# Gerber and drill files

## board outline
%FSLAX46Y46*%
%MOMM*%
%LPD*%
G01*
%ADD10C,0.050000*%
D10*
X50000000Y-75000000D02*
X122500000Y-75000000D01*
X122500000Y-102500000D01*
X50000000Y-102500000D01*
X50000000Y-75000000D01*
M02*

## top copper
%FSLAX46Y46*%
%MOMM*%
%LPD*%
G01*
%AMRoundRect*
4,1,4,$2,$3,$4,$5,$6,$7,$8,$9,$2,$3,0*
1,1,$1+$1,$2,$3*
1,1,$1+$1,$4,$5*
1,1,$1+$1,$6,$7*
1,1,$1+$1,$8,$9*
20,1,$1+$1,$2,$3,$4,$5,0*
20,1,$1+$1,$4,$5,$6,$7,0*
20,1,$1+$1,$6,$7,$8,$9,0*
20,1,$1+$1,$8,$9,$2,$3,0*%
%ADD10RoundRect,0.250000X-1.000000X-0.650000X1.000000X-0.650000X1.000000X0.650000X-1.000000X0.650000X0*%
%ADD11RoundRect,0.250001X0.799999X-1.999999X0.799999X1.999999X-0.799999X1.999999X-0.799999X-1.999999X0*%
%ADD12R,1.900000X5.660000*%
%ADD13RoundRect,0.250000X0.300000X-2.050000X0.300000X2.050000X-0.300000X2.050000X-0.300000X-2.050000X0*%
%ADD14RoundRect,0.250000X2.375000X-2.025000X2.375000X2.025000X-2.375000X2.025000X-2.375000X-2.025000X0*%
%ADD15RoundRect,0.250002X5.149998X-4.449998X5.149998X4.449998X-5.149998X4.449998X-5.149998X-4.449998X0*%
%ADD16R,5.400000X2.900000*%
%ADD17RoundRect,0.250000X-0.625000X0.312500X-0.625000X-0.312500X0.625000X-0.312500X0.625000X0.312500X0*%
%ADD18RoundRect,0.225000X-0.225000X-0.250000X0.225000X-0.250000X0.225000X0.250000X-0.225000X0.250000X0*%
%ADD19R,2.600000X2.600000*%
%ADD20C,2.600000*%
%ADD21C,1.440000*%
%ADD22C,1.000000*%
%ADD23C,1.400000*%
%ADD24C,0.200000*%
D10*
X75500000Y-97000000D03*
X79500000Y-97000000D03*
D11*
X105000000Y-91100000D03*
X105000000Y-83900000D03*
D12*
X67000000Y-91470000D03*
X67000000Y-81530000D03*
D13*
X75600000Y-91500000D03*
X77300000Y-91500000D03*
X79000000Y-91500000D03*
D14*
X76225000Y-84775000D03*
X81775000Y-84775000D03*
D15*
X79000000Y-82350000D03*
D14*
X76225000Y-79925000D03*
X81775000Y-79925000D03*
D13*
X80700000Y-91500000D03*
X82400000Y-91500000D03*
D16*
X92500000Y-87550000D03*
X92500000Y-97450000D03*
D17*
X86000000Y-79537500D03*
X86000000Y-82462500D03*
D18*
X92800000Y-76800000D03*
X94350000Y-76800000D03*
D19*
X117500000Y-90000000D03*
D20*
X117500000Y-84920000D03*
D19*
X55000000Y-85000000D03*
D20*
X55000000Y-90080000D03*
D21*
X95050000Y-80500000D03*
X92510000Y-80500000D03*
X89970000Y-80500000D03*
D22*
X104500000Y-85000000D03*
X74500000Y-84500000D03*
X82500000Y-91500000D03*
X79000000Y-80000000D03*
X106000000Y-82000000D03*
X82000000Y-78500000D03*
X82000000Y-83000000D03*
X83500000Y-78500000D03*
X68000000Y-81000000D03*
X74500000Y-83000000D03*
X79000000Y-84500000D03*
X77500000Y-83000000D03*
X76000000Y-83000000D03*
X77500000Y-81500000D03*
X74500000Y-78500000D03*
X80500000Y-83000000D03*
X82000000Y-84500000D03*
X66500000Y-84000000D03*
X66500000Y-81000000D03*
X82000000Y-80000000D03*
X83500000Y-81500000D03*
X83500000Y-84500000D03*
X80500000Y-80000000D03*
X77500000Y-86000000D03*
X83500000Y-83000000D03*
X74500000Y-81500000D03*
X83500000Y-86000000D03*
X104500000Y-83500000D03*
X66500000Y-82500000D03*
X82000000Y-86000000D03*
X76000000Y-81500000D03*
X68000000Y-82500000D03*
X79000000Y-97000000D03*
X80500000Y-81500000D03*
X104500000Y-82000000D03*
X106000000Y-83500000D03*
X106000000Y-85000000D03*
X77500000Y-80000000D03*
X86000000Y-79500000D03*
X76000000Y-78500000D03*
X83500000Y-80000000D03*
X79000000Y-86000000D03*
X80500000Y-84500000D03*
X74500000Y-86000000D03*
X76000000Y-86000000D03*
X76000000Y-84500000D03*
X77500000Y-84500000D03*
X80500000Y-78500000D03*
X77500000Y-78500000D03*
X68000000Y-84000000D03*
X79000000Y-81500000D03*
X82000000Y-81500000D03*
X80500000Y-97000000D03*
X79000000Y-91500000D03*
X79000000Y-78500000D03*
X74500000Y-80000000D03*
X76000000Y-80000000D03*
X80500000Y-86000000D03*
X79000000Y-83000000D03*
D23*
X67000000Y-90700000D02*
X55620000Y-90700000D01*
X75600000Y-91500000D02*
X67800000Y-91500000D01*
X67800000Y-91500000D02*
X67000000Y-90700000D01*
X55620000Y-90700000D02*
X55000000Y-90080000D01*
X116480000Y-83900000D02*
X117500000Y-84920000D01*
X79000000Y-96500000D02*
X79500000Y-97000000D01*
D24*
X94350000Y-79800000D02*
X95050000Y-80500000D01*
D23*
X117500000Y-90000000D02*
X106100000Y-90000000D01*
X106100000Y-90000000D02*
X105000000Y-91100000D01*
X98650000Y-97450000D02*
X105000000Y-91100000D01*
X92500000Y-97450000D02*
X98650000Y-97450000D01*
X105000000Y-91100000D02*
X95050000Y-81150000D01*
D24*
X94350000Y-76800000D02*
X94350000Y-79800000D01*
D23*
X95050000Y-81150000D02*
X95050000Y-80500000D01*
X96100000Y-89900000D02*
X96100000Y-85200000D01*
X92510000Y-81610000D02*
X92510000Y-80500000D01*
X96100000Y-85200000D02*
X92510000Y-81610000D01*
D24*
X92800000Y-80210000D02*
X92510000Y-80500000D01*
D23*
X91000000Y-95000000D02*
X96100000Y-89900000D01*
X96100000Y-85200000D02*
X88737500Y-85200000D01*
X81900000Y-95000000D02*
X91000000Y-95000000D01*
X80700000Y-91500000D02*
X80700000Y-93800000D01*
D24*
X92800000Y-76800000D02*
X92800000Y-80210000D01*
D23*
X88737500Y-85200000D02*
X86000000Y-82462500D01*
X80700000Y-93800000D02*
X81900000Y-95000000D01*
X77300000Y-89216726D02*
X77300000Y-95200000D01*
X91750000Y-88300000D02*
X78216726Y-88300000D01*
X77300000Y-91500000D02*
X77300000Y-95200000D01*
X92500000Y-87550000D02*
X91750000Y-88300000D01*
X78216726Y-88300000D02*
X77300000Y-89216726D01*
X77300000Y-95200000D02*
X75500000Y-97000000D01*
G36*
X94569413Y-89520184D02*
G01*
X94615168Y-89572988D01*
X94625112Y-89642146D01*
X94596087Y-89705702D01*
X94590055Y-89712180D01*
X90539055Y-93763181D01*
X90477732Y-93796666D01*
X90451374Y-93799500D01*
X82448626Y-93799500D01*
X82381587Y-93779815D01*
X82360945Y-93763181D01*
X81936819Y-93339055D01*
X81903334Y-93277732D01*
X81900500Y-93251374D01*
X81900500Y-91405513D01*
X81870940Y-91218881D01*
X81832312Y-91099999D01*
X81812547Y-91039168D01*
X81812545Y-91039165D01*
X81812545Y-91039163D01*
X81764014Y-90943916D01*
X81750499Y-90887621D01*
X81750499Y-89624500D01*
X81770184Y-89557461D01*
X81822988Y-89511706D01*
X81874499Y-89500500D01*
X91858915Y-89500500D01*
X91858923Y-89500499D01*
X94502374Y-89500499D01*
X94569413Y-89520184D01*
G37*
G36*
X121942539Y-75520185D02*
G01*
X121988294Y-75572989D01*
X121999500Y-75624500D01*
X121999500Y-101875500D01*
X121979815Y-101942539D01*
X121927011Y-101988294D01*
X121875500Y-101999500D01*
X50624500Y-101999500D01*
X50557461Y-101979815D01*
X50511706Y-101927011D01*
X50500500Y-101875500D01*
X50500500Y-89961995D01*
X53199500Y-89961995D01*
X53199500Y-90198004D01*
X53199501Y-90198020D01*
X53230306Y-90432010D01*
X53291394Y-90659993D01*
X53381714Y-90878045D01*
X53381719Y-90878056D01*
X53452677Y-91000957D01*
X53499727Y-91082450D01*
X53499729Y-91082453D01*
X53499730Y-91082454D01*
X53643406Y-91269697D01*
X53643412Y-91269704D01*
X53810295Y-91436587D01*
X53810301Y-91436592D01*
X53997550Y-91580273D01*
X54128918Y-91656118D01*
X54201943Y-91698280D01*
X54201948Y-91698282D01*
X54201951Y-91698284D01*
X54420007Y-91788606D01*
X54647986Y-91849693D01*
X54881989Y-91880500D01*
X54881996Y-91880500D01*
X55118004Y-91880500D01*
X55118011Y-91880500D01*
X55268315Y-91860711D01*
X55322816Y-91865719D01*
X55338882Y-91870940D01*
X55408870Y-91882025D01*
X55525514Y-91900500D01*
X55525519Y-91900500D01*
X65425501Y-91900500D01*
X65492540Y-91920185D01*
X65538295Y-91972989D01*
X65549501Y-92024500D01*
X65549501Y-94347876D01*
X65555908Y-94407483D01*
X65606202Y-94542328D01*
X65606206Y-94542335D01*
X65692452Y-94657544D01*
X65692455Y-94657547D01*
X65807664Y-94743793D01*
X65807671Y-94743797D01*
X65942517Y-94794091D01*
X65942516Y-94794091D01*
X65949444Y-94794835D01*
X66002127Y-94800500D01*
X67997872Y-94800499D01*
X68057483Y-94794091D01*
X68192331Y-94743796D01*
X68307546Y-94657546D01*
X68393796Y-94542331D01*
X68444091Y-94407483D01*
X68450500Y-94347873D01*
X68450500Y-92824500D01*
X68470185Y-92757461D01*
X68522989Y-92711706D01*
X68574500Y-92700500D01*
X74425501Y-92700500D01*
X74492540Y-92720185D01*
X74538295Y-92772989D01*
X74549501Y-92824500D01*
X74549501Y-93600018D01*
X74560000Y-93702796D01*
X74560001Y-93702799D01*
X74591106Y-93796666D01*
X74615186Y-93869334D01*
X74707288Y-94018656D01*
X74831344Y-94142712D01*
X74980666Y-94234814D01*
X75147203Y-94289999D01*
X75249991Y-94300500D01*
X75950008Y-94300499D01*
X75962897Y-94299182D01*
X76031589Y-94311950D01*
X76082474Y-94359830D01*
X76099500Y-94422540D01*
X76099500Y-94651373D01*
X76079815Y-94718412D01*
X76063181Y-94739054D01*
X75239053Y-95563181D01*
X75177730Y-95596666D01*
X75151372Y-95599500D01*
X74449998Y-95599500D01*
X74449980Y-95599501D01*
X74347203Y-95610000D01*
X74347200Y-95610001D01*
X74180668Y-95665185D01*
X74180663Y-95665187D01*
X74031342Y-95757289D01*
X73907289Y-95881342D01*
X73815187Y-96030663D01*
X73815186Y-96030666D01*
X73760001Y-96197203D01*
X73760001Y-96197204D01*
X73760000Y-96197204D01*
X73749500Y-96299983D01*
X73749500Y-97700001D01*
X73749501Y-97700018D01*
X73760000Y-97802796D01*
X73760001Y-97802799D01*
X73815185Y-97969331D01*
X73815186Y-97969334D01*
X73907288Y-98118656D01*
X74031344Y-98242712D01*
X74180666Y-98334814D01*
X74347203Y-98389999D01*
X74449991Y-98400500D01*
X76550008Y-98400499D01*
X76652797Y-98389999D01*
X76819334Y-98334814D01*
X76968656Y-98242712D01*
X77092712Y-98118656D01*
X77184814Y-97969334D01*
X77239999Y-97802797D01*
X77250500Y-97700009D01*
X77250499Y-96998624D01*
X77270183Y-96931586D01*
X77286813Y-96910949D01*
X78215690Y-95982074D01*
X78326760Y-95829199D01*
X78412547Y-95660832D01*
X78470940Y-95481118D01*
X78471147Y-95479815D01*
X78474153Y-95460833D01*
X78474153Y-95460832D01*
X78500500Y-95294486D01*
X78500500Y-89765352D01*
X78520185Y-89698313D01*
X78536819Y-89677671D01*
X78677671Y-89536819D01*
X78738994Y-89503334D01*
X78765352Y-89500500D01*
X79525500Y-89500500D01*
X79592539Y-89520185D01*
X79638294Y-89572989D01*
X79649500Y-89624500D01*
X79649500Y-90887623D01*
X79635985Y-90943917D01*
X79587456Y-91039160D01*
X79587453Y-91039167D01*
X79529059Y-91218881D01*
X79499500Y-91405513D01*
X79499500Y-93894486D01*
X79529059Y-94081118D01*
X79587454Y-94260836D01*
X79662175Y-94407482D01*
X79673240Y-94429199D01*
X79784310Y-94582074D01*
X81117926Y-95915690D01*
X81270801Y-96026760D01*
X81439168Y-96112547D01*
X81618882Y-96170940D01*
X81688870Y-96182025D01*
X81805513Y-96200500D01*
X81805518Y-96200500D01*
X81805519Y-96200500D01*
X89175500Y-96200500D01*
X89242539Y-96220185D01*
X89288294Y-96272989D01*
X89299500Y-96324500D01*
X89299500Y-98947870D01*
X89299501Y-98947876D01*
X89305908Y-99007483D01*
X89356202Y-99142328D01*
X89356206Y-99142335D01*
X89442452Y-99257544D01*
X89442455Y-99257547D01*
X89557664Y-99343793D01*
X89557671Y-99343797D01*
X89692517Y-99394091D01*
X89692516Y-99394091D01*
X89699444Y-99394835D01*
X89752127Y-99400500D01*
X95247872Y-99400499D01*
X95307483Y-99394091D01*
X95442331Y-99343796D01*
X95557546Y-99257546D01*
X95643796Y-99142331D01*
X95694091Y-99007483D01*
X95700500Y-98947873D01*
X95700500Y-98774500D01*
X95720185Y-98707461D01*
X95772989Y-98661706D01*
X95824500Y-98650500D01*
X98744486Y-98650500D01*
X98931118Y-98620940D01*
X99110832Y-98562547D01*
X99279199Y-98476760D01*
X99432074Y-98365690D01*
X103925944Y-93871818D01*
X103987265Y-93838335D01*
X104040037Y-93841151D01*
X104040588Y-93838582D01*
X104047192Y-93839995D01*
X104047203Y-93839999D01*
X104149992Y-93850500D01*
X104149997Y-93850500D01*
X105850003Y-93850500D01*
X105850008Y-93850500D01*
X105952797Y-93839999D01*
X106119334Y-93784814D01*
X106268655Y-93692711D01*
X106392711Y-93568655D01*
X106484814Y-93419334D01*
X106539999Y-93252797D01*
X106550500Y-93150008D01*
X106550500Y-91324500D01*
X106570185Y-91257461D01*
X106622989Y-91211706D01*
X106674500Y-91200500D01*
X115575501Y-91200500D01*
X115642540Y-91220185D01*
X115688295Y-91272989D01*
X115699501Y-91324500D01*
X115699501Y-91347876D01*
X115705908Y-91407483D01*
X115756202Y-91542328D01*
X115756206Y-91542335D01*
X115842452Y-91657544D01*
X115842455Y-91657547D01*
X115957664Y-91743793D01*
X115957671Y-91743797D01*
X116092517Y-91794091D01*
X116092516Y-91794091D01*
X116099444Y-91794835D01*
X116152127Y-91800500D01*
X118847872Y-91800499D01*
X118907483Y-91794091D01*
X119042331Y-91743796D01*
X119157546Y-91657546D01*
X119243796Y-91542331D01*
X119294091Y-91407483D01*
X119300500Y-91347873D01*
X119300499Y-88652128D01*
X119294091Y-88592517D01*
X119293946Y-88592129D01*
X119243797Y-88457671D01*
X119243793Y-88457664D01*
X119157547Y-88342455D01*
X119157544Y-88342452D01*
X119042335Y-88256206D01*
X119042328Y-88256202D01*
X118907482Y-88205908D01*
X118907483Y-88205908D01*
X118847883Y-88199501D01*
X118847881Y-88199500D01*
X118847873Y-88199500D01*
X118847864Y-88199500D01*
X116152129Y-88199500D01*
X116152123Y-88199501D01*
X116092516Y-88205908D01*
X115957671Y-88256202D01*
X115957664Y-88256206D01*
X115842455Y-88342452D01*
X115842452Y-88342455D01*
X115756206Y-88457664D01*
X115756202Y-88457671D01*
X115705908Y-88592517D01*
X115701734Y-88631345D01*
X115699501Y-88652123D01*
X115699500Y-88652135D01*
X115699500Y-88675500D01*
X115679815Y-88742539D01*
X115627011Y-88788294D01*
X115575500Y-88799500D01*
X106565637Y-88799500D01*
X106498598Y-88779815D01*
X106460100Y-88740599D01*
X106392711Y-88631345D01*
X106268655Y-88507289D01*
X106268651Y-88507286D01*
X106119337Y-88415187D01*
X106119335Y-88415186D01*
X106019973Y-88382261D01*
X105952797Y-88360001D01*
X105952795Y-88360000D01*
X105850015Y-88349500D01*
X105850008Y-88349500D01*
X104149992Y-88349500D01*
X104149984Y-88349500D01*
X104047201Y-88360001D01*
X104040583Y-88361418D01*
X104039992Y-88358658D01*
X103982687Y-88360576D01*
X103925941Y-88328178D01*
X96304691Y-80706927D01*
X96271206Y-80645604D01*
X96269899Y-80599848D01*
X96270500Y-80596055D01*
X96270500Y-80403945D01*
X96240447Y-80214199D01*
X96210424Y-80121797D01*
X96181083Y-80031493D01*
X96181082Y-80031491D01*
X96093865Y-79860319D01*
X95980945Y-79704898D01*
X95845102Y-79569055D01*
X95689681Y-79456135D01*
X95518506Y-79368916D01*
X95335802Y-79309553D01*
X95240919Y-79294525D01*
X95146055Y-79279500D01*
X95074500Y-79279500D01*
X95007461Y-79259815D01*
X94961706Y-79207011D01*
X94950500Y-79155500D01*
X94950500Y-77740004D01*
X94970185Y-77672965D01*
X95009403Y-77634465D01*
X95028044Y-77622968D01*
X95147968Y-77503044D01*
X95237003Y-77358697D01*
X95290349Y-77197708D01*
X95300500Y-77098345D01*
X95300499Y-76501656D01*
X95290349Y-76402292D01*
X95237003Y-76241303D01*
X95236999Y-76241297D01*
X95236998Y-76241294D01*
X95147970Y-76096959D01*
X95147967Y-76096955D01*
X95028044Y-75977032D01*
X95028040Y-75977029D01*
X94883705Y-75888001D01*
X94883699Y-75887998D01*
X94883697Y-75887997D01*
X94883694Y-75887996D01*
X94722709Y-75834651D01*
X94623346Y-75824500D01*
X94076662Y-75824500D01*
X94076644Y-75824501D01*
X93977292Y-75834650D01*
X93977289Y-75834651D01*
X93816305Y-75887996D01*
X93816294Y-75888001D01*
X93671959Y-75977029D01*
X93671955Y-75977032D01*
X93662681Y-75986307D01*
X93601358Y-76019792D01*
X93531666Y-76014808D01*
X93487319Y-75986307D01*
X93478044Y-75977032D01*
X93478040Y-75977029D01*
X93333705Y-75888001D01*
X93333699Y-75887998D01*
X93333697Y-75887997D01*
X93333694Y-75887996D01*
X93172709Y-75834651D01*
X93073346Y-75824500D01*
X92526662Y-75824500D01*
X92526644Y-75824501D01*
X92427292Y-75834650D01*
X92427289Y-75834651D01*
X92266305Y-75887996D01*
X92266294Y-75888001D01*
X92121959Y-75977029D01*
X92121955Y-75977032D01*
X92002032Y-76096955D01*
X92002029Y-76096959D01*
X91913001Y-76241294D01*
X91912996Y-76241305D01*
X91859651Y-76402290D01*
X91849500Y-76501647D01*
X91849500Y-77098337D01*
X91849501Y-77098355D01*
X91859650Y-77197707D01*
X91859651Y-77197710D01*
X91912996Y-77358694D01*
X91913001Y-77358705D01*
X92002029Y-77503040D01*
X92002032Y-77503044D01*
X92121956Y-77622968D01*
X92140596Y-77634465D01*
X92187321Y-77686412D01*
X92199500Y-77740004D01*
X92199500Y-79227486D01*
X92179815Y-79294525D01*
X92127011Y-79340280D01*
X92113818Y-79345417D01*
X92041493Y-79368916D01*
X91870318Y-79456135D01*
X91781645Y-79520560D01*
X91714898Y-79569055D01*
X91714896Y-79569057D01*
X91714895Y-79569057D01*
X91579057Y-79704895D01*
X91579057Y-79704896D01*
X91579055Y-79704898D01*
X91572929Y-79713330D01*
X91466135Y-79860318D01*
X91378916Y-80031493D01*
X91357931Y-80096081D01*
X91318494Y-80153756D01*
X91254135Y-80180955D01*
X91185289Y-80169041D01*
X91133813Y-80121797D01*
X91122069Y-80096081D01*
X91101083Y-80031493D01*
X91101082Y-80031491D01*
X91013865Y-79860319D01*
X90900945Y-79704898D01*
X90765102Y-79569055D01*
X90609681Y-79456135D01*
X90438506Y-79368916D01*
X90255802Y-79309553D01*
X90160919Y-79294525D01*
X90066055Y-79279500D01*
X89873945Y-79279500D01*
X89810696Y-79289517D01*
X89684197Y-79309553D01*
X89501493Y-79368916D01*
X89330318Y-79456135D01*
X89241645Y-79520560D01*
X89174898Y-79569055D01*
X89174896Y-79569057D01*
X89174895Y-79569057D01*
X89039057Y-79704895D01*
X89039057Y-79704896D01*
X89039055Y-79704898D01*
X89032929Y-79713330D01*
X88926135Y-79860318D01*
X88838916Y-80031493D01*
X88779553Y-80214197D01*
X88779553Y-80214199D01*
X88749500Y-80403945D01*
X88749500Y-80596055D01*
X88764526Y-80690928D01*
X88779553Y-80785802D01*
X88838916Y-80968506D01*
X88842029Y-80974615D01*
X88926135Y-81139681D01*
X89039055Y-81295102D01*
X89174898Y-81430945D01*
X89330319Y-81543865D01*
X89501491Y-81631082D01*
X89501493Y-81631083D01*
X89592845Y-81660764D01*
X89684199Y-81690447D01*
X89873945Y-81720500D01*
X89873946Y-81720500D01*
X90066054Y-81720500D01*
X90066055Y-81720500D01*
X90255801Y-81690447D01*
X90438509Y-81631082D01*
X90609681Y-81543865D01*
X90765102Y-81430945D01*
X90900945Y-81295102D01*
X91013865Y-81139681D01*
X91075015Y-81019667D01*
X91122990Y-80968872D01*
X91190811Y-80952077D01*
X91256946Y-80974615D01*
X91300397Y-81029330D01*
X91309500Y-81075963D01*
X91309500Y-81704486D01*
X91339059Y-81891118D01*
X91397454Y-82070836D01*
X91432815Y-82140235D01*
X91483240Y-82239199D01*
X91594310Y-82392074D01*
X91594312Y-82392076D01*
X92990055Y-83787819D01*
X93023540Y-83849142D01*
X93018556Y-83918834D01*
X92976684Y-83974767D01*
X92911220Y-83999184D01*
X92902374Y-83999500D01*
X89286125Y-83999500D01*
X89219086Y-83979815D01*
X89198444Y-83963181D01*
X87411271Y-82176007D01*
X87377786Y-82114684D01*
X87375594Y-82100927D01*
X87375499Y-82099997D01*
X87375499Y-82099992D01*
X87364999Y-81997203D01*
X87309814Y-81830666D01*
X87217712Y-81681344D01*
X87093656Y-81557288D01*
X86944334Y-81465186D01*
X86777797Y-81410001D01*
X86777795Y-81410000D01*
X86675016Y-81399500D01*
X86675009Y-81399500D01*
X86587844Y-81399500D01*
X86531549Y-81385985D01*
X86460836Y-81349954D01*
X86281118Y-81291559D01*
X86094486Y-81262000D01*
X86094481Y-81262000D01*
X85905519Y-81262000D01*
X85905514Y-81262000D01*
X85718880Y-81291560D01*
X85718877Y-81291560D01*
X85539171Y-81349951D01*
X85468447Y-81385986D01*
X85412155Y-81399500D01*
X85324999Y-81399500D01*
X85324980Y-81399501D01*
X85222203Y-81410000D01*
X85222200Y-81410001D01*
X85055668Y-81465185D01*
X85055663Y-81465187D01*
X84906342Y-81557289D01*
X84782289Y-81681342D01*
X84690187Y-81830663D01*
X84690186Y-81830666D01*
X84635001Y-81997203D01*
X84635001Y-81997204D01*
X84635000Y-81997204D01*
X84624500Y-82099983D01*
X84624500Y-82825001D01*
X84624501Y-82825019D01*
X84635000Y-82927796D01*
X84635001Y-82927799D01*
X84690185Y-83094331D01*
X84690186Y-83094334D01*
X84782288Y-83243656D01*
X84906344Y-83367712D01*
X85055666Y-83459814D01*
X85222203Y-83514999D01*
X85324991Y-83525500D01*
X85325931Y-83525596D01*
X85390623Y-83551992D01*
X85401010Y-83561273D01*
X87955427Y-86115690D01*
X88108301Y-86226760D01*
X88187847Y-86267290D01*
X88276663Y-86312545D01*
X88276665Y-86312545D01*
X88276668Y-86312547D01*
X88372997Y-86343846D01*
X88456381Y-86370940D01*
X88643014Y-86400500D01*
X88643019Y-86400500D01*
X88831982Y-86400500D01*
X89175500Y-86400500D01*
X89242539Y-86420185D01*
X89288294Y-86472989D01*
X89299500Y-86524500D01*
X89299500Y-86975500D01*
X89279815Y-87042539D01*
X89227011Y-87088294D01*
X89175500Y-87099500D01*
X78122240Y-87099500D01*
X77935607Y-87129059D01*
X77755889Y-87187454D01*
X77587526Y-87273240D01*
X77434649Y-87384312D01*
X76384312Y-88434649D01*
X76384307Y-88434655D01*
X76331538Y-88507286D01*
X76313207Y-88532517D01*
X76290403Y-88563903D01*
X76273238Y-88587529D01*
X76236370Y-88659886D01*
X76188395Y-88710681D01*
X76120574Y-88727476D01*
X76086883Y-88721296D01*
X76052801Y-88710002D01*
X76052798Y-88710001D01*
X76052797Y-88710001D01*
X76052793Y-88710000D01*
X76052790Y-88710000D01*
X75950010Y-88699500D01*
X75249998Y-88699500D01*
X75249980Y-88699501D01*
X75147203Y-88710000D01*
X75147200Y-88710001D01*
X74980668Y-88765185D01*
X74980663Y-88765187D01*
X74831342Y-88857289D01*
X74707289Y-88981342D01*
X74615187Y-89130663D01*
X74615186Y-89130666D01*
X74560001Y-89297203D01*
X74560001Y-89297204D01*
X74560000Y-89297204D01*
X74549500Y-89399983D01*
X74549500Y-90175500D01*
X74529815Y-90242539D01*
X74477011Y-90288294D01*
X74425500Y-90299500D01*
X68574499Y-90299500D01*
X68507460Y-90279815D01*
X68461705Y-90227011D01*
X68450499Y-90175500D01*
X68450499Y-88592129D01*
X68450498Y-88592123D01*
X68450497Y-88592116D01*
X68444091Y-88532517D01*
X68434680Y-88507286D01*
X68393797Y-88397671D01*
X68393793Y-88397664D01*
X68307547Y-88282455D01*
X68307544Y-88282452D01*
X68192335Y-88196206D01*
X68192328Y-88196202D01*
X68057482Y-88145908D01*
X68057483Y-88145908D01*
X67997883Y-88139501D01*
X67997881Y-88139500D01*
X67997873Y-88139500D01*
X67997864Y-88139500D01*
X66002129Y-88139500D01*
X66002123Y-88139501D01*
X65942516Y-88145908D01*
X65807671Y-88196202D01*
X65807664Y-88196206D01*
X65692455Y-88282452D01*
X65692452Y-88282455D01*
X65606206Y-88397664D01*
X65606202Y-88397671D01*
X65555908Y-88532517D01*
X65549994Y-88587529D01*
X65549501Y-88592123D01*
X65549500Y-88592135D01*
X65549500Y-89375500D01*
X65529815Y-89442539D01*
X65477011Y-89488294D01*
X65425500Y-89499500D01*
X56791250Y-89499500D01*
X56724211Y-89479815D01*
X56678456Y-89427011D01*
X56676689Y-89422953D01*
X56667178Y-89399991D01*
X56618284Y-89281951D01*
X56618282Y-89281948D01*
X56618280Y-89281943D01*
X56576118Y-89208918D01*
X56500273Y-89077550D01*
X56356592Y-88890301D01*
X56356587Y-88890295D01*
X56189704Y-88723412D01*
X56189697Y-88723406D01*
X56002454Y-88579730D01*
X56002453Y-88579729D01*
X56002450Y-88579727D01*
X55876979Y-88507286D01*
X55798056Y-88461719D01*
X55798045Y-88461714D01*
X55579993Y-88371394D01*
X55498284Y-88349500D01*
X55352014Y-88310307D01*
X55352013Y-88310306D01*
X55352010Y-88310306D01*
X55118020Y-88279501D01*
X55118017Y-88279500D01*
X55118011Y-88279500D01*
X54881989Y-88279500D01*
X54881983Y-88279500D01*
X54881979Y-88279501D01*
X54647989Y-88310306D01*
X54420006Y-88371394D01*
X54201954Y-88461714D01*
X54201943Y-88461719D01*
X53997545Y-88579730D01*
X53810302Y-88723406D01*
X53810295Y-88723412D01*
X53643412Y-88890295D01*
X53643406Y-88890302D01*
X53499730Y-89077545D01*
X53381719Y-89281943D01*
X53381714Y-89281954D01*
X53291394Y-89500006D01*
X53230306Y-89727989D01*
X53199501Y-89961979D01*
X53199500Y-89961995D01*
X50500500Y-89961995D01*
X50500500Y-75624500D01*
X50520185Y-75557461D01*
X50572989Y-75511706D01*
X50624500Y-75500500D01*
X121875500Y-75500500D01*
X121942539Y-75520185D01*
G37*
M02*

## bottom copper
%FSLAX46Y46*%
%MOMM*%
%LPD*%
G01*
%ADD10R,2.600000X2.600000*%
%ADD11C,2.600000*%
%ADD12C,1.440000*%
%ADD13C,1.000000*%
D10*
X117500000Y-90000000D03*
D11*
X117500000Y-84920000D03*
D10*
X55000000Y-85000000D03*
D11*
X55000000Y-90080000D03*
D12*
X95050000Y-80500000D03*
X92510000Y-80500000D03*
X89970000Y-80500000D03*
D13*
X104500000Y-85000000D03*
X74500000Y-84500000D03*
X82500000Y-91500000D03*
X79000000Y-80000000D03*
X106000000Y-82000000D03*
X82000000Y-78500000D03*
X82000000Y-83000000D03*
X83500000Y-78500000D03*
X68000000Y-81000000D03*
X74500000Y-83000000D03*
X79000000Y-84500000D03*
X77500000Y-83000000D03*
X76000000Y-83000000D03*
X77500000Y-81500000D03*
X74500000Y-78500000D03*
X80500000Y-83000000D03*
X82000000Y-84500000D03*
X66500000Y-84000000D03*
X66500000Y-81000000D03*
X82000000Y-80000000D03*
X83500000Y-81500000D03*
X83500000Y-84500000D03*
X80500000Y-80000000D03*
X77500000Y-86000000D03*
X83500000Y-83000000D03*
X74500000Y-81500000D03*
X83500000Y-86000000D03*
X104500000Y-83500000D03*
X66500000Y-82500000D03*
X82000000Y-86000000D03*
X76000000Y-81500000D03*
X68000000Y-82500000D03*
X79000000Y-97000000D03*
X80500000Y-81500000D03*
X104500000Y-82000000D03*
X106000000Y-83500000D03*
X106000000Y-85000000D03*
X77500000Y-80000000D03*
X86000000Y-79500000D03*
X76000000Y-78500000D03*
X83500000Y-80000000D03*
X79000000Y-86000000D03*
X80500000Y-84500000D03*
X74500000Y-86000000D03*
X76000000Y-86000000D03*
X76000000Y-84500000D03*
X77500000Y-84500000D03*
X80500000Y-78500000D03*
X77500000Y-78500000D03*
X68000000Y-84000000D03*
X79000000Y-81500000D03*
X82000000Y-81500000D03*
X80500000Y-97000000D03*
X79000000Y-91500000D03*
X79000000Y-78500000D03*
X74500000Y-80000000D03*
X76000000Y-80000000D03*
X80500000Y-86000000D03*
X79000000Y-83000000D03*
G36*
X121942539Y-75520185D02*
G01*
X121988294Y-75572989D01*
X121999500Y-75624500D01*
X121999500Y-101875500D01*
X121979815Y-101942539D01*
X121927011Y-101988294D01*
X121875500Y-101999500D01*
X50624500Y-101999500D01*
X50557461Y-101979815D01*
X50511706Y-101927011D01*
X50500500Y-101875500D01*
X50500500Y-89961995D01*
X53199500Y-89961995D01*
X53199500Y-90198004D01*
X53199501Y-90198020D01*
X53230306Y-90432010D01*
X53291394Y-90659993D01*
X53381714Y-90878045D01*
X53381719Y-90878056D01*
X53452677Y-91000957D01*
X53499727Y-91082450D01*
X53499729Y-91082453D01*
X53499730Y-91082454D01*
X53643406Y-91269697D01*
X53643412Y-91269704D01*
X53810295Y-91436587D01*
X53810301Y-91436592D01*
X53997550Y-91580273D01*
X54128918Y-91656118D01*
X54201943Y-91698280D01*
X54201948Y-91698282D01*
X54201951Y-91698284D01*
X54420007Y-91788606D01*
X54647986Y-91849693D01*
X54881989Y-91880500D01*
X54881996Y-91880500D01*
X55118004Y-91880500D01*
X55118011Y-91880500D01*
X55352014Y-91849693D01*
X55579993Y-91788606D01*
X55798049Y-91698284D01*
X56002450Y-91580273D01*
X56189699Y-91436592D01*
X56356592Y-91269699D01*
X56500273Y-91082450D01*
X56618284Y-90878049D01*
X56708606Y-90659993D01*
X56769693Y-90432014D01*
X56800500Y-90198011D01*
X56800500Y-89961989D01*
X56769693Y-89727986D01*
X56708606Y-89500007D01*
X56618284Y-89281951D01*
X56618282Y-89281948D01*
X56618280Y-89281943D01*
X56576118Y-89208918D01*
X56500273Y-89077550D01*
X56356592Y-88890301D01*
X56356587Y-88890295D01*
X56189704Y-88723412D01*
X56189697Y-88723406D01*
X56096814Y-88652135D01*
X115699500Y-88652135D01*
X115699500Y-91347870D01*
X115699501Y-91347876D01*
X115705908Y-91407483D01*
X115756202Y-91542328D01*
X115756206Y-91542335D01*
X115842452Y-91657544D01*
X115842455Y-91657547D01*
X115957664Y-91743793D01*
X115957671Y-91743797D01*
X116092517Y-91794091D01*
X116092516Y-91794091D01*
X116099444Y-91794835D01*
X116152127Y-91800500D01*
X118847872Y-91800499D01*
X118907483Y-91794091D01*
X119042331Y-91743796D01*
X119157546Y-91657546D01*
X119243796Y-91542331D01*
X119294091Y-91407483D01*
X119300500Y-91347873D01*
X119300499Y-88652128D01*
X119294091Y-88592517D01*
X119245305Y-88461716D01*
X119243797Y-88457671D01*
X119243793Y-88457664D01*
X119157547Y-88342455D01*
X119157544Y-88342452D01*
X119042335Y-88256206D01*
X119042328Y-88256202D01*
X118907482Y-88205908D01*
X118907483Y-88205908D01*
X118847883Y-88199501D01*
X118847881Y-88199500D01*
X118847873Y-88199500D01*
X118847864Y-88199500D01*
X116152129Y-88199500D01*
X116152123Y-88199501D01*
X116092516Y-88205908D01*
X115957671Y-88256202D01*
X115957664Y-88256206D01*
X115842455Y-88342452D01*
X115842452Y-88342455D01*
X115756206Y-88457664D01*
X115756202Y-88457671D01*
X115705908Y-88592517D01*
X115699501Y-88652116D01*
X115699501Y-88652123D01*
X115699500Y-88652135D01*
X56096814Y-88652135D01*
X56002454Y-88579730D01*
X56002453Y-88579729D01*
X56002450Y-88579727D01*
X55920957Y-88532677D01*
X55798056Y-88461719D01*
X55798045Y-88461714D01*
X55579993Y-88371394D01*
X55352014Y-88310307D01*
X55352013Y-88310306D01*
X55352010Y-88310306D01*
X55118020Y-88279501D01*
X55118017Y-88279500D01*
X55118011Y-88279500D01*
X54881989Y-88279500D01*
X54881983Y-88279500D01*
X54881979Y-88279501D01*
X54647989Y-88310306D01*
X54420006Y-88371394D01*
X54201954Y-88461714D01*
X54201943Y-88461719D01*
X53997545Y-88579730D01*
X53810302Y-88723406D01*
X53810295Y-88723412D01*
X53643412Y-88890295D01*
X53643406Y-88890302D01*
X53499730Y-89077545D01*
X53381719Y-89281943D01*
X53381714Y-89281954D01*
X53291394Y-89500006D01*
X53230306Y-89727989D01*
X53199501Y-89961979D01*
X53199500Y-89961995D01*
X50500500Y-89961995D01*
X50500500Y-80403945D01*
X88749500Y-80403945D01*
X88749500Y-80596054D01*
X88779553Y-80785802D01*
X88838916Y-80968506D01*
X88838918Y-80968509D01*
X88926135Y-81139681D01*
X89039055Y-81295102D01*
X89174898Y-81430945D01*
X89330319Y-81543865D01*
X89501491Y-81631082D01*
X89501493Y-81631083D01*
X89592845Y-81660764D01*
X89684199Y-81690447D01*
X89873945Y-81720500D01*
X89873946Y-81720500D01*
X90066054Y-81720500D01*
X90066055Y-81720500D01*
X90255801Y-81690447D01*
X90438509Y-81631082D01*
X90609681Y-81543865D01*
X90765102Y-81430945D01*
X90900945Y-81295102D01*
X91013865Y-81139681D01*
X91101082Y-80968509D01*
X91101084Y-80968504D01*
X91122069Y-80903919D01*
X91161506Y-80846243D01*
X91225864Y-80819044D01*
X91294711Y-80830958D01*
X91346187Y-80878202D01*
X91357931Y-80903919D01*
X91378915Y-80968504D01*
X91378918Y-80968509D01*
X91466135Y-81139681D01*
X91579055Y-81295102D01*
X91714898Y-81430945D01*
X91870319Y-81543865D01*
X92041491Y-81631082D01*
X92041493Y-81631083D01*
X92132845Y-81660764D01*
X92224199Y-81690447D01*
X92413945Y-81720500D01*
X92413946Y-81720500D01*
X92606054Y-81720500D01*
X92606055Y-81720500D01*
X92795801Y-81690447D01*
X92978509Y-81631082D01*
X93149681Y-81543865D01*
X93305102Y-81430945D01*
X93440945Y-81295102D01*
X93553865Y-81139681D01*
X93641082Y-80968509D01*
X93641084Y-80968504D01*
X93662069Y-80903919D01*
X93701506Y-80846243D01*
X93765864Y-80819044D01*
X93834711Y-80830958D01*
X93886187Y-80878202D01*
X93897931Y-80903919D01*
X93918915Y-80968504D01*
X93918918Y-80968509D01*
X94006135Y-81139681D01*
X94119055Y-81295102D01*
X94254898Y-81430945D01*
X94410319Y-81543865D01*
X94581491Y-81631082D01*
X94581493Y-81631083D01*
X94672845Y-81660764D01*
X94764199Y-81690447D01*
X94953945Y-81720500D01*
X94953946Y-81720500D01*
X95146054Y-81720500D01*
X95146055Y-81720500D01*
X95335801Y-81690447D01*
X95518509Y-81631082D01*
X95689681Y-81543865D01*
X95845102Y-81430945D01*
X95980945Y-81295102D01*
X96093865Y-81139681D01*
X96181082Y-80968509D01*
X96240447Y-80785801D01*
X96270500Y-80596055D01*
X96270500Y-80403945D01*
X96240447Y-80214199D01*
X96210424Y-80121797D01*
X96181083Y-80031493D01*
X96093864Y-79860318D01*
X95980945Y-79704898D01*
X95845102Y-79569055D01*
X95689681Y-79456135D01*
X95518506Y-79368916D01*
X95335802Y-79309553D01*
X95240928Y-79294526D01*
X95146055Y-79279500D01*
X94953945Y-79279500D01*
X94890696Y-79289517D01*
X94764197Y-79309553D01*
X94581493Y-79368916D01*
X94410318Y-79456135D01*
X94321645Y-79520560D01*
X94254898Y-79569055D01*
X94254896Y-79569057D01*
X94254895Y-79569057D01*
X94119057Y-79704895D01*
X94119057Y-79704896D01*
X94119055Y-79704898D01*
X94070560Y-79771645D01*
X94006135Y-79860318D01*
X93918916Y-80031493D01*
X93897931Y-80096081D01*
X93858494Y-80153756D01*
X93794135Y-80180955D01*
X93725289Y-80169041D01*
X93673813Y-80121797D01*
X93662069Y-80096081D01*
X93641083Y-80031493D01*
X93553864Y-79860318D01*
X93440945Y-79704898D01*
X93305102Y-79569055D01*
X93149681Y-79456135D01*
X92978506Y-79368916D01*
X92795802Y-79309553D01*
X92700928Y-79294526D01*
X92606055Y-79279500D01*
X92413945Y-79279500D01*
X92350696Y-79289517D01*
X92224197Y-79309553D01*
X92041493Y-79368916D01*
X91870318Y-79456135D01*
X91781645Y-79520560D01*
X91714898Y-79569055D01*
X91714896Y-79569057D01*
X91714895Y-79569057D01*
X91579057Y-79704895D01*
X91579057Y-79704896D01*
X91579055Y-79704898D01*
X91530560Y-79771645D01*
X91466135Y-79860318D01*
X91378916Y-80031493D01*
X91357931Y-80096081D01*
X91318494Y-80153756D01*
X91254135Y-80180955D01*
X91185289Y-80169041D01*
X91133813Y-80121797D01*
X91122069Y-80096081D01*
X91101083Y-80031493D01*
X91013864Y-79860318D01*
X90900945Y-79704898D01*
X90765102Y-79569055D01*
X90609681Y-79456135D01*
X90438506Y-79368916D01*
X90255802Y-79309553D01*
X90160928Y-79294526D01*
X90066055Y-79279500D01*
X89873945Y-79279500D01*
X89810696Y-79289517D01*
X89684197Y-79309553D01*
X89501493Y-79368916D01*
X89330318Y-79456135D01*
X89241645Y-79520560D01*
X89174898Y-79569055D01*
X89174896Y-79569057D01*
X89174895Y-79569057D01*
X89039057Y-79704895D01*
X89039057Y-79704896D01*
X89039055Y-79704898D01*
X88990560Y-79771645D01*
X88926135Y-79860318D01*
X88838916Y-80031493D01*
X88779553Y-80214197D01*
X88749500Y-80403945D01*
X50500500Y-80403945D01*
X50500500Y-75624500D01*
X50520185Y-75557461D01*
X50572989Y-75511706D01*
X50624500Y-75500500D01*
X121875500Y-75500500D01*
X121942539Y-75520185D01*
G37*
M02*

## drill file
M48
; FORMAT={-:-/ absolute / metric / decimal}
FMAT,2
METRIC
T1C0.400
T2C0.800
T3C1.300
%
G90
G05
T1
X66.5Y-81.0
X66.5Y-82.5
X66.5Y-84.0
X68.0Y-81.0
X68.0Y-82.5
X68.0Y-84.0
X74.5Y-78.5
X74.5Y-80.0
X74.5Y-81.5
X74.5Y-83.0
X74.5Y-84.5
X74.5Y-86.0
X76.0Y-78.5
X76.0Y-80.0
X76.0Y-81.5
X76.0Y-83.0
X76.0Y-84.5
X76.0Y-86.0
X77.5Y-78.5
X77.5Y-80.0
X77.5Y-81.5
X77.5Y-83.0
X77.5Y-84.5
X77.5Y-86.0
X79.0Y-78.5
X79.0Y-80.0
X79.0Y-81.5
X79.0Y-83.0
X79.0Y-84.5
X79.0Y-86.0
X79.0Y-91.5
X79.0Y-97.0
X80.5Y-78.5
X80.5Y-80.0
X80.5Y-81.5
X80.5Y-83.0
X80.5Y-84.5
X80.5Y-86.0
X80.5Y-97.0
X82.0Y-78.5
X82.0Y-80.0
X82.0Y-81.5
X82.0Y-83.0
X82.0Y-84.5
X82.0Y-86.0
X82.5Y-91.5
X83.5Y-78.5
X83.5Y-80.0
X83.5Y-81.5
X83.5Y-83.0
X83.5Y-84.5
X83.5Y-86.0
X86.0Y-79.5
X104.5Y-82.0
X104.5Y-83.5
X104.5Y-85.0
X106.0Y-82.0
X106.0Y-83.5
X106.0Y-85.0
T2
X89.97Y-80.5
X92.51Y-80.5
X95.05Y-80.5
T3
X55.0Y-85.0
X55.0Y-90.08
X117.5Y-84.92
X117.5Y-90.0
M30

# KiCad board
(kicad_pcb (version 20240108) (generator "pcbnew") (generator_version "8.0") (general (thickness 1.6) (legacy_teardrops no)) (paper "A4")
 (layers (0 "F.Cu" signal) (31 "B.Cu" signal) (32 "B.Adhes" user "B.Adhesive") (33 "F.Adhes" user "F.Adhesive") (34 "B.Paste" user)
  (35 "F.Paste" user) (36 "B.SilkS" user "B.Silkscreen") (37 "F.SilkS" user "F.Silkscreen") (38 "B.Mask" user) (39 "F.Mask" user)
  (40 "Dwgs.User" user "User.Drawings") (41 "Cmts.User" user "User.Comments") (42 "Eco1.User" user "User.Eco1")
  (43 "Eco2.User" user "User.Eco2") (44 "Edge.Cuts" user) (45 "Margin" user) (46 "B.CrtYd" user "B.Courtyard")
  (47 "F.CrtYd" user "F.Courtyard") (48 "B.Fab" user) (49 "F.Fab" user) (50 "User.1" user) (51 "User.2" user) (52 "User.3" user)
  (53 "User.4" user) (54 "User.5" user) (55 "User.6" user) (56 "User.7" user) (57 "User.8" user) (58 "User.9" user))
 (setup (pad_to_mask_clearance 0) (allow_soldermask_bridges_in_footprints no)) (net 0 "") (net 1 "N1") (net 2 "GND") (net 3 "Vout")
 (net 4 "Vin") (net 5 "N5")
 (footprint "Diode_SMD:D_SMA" (layer "F.Cu") (at 77.5 97)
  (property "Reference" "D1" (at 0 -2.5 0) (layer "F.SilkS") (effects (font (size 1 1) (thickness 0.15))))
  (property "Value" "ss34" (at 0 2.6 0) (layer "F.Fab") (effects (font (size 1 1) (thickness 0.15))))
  (pad "1" smd roundrect (at -2 0) (size 2.5 1.8) (layers "F.Cu" "F.Paste" "F.Mask") (roundrect_rratio 0.1388888889) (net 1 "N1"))
  (pad "2" smd roundrect (at 2 0) (size 2.5 1.8) (layers "F.Cu" "F.Paste" "F.Mask") (roundrect_rratio 0.1388888889) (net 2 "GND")))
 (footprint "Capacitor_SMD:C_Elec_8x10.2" (layer "F.Cu") (at 105 87.5 90)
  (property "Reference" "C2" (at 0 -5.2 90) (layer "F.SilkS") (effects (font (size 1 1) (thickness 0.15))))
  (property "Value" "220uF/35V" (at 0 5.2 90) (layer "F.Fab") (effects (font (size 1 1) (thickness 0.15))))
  (pad "1" smd roundrect (at -3.6 0 90) (size 4.5 2.1) (layers "F.Cu" "F.Paste" "F.Mask") (roundrect_rratio 0.119048) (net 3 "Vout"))
  (pad "2" smd roundrect (at 3.6 0 90) (size 4.5 2.1) (layers "F.Cu" "F.Paste" "F.Mask") (roundrect_rratio 0.119048) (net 2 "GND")))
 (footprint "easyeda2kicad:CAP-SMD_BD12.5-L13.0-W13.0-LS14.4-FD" (layer "F.Cu") (at 67 86.5 90)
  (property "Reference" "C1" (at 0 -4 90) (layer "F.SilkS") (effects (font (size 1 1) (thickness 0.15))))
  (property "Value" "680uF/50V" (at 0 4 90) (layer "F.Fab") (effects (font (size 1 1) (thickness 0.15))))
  (pad "1" smd rect (at -4.97 0 90) (size 5.66 1.9) (layers "F.Cu" "F.Paste" "F.Mask") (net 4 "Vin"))
  (pad "2" smd rect (at 4.97 0 90) (size 5.66 1.9) (layers "F.Cu" "F.Paste" "F.Mask") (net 2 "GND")))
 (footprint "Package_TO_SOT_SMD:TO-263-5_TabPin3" (layer "F.Cu") (at 79 83.85 90)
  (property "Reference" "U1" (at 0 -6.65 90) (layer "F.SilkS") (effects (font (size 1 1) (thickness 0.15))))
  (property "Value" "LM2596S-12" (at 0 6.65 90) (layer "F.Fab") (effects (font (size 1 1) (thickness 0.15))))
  (pad "1" smd roundrect (at -7.65 -3.4 90) (size 4.6 1.1) (layers "F.Cu" "F.Paste" "F.Mask") (roundrect_rratio 0.227273) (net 4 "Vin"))
  (pad "2" smd roundrect (at -7.65 -1.7 90) (size 4.6 1.1) (layers "F.Cu" "F.Paste" "F.Mask") (roundrect_rratio 0.227273) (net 1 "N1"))
  (pad "3" smd roundrect (at -7.65 0 90) (size 4.6 1.1) (layers "F.Cu" "F.Paste" "F.Mask") (roundrect_rratio 0.227273) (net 2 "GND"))
  (pad "3" smd roundrect (at -0.925 -2.775 90) (size 4.55 5.25) (layers "F.Cu" "F.Paste") (roundrect_rratio 0.054945) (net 2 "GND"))
  (pad "3" smd roundrect (at -0.925 2.775 90) (size 4.55 5.25) (layers "F.Cu" "F.Paste") (roundrect_rratio 0.054945) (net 2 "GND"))
  (pad "3" smd roundrect (at 1.5 0 90) (size 9.4 10.8) (layers "F.Cu" "F.Mask") (roundrect_rratio 0.026596) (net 2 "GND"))
  (pad "3" smd roundrect (at 3.925 -2.775 90) (size 4.55 5.25) (layers "F.Cu" "F.Paste") (roundrect_rratio 0.054945) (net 2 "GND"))
  (pad "3" smd roundrect (at 3.925 2.775 90) (size 4.55 5.25) (layers "F.Cu" "F.Paste") (roundrect_rratio 0.054945) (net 2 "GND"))
  (pad "4" smd roundrect (at -7.65 1.7 90) (size 4.6 1.1) (layers "F.Cu" "F.Paste" "F.Mask") (roundrect_rratio 0.227273) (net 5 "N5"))
  (pad "5" smd roundrect (at -7.65 3.4 90) (size 4.6 1.1) (layers "F.Cu" "F.Paste" "F.Mask") (roundrect_rratio 0.227273) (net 2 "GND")))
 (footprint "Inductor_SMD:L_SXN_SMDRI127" (layer "F.Cu") (at 92.5 92.5 -90)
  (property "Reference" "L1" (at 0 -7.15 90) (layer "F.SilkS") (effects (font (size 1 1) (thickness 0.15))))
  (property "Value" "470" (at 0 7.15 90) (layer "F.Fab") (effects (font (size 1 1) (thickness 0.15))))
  (pad "1" smd rect (at -4.95 0 270) (size 2.9 5.4) (layers "F.Cu" "F.Paste" "F.Mask") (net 1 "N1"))
  (pad "2" smd rect (at 4.95 0 270) (size 2.9 5.4) (layers "F.Cu" "F.Paste" "F.Mask") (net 3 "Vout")))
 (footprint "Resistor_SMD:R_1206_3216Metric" (layer "F.Cu") (at 86 81 -90)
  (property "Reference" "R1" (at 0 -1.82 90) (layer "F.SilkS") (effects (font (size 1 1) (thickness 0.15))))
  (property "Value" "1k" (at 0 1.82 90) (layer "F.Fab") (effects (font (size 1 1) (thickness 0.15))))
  (pad "1" smd roundrect (at -1.4625 0 270) (size 1.125 1.75) (layers "F.Cu" "F.Paste" "F.Mask") (roundrect_rratio 0.222222) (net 2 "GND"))
  (pad "2" smd roundrect (at 1.4625 0 270) (size 1.125 1.75) (layers "F.Cu" "F.Paste" "F.Mask") (roundrect_rratio 0.222222) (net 5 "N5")))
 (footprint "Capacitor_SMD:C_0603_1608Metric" (layer "F.Cu") (at 93.575 76.8)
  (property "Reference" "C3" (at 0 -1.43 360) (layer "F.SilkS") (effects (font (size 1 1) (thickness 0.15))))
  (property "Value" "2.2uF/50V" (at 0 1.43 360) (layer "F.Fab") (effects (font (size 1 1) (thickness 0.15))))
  (pad "1" smd roundrect (at -0.775 0) (size 0.9 0.95) (layers "F.Cu" "F.Paste" "F.Mask") (roundrect_rratio 0.25) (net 5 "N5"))
  (pad "2" smd roundrect (at 0.775 0) (size 0.9 0.95) (layers "F.Cu" "F.Paste" "F.Mask") (roundrect_rratio 0.25) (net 3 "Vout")))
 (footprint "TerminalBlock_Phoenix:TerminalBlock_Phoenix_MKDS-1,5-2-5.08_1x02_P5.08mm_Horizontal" (layer "F.Cu") (at 117.5 90 90)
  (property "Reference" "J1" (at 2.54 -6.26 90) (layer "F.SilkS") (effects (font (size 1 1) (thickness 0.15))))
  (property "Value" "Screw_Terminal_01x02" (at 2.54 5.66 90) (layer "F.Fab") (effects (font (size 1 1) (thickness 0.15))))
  (pad "1" thru_hole rect (at 0 0 90) (size 2.6 2.6) (drill 1.3) (layers "*.Cu" "*.Mask") (remove_unused_layers no) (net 3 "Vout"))
  (pad "2" thru_hole circle (at 5.08 0 90) (size 2.6 2.6) (drill 1.3) (layers "*.Cu" "*.Mask") (remove_unused_layers no) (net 2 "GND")))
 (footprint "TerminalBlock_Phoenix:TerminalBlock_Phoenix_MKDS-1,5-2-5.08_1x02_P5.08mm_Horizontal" (layer "F.Cu") (at 55 85 -90)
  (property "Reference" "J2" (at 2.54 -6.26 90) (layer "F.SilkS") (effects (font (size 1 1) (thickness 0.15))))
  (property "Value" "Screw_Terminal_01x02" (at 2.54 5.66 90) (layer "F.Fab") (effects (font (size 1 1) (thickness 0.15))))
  (pad "1" thru_hole rect (at 0 0 270) (size 2.6 2.6) (drill 1.3) (layers "*.Cu" "*.Mask") (remove_unused_layers no) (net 2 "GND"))
  (pad "2" thru_hole circle (at 5.08 0 270) (size 2.6 2.6) (drill 1.3) (layers "*.Cu" "*.Mask") (remove_unused_layers no) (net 4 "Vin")))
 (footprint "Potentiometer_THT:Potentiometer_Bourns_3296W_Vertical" (layer "F.Cu") (at 95.05 80.5)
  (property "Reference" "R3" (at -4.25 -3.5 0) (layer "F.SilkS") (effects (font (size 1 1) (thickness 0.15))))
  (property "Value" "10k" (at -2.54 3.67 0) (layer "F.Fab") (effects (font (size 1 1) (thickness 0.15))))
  (pad "1" thru_hole circle (at 0 0) (size 1.44 1.44) (drill 0.8) (layers "*.Cu" "*.Mask") (remove_unused_layers no) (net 3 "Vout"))
  (pad "2" thru_hole circle (at -2.54 0) (size 1.44 1.44) (drill 0.8) (layers "*.Cu" "*.Mask") (remove_unused_layers no) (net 5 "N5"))
  (pad "3" thru_hole circle (at -5.08 0) (size 1.44 1.44) (drill 0.8) (layers "*.Cu" "*.Mask") (remove_unused_layers no)))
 (gr_rect (start 50 75) (end 122.5 102.5) (stroke (width 0.05) (type default)) (fill none) (layer "Edge.Cuts"))
 (segment (start 67 90.7) (end 55.62 90.7) (width 1.4) (layer "F.Cu") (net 4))
 (segment (start 75.6 91.5) (end 67.8 91.5) (width 1.4) (layer "F.Cu") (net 4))
 (segment (start 67.8 91.5) (end 67 90.7) (width 1.4) (layer "F.Cu") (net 4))
 (segment (start 55.62 90.7) (end 55 90.08) (width 1.4) (layer "F.Cu") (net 4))
 (segment (start 116.48 83.9) (end 117.5 84.92) (width 1.4) (layer "F.Cu") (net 2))
 (segment (start 79 96.5) (end 79.5 97) (width 1.4) (layer "F.Cu") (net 2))
 (via (at 104.5 85) (size 1) (drill 0.4) (layers "F.Cu" "B.Cu") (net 2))
 (via (at 74.5 84.5) (size 1) (drill 0.4) (layers "F.Cu" "B.Cu") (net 2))
 (via (at 82.5 91.5) (size 1) (drill 0.4) (layers "F.Cu" "B.Cu") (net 2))
 (via (at 79 80) (size 1) (drill 0.4) (layers "F.Cu" "B.Cu") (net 2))
 (via (at 106 82) (size 1) (drill 0.4) (layers "F.Cu" "B.Cu") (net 2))
 (via (at 82 78.5) (size 1) (drill 0.4) (layers "F.Cu" "B.Cu") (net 2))
 (via (at 82 83) (size 1) (drill 0.4) (layers "F.Cu" "B.Cu") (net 2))
 (via (at 83.5 78.5) (size 1) (drill 0.4) (layers "F.Cu" "B.Cu") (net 2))
 (via (at 68 81) (size 1) (drill 0.4) (layers "F.Cu" "B.Cu") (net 2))
 (via (at 74.5 83) (size 1) (drill 0.4) (layers "F.Cu" "B.Cu") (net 2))
 (via (at 79 84.5) (size 1) (drill 0.4) (layers "F.Cu" "B.Cu") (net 2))
 (via (at 77.5 83) (size 1) (drill 0.4) (layers "F.Cu" "B.Cu") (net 2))
 (via (at 76 83) (size 1) (drill 0.4) (layers "F.Cu" "B.Cu") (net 2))
 (via (at 77.5 81.5) (size 1) (drill 0.4) (layers "F.Cu" "B.Cu") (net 2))
 (via (at 74.5 78.5) (size 1) (drill 0.4) (layers "F.Cu" "B.Cu") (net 2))
 (via (at 80.5 83) (size 1) (drill 0.4) (layers "F.Cu" "B.Cu") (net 2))
 (via (at 82 84.5) (size 1) (drill 0.4) (layers "F.Cu" "B.Cu") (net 2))
 (via (at 66.5 84) (size 1) (drill 0.4) (layers "F.Cu" "B.Cu") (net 2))
 (via (at 66.5 81) (size 1) (drill 0.4) (layers "F.Cu" "B.Cu") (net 2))
 (via (at 82 80) (size 1) (drill 0.4) (layers "F.Cu" "B.Cu") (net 2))
 (via (at 83.5 81.5) (size 1) (drill 0.4) (layers "F.Cu" "B.Cu") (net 2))
 (via (at 83.5 84.5) (size 1) (drill 0.4) (layers "F.Cu" "B.Cu") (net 2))
 (via (at 80.5 80) (size 1) (drill 0.4) (layers "F.Cu" "B.Cu") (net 2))
 (via (at 77.5 86) (size 1) (drill 0.4) (layers "F.Cu" "B.Cu") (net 2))
 (via (at 83.5 83) (size 1) (drill 0.4) (layers "F.Cu" "B.Cu") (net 2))
 (via (at 74.5 81.5) (size 1) (drill 0.4) (layers "F.Cu" "B.Cu") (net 2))
 (via (at 83.5 86) (size 1) (drill 0.4) (layers "F.Cu" "B.Cu") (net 2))
 (via (at 104.5 83.5) (size 1) (drill 0.4) (layers "F.Cu" "B.Cu") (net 2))
 (via (at 66.5 82.5) (size 1) (drill 0.4) (layers "F.Cu" "B.Cu") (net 2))
 (via (at 82 86) (size 1) (drill 0.4) (layers "F.Cu" "B.Cu") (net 2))
 (via (at 76 81.5) (size 1) (drill 0.4) (layers "F.Cu" "B.Cu") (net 2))
 (via (at 68 82.5) (size 1) (drill 0.4) (layers "F.Cu" "B.Cu") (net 2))
 (via (at 79 97) (size 1) (drill 0.4) (layers "F.Cu" "B.Cu") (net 2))
 (via (at 80.5 81.5) (size 1) (drill 0.4) (layers "F.Cu" "B.Cu") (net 2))
 (via (at 104.5 82) (size 1) (drill 0.4) (layers "F.Cu" "B.Cu") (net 2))
 (via (at 106 83.5) (size 1) (drill 0.4) (layers "F.Cu" "B.Cu") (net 2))
 (via (at 106 85) (size 1) (drill 0.4) (layers "F.Cu" "B.Cu") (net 2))
 (via (at 77.5 80) (size 1) (drill 0.4) (layers "F.Cu" "B.Cu") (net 2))
 (via (at 86 79.5) (size 1) (drill 0.4) (layers "F.Cu" "B.Cu") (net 2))
 (via (at 76 78.5) (size 1) (drill 0.4) (layers "F.Cu" "B.Cu") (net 2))
 (via (at 83.5 80) (size 1) (drill 0.4) (layers "F.Cu" "B.Cu") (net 2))
 (via (at 79 86) (size 1) (drill 0.4) (layers "F.Cu" "B.Cu") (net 2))
 (via (at 80.5 84.5) (size 1) (drill 0.4) (layers "F.Cu" "B.Cu") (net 2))
 (via (at 74.5 86) (size 1) (drill 0.4) (layers "F.Cu" "B.Cu") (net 2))
 (via (at 76 86) (size 1) (drill 0.4) (layers "F.Cu" "B.Cu") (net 2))
 (via (at 76 84.5) (size 1) (drill 0.4) (layers "F.Cu" "B.Cu") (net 2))
 (via (at 77.5 84.5) (size 1) (drill 0.4) (layers "F.Cu" "B.Cu") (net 2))
 (via (at 80.5 78.5) (size 1) (drill 0.4) (layers "F.Cu" "B.Cu") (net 2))
 (via (at 77.5 78.5) (size 1) (drill 0.4) (layers "F.Cu" "B.Cu") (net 2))
 (via (at 68 84) (size 1) (drill 0.4) (layers "F.Cu" "B.Cu") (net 2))
 (via (at 79 81.5) (size 1) (drill 0.4) (layers "F.Cu" "B.Cu") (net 2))
 (via (at 82 81.5) (size 1) (drill 0.4) (layers "F.Cu" "B.Cu") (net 2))
 (via (at 80.5 97) (size 1) (drill 0.4) (layers "F.Cu" "B.Cu") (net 2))
 (via (at 79 91.5) (size 1) (drill 0.4) (layers "F.Cu" "B.Cu") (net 2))
 (via (at 79 78.5) (size 1) (drill 0.4) (layers "F.Cu" "B.Cu") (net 2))
 (via (at 74.5 80) (size 1) (drill 0.4) (layers "F.Cu" "B.Cu") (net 2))
 (via (at 76 80) (size 1) (drill 0.4) (layers "F.Cu" "B.Cu") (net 2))
 (via (at 80.5 86) (size 1) (drill 0.4) (layers "F.Cu" "B.Cu") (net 2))
 (via (at 79 83) (size 1) (drill 0.4) (layers "F.Cu" "B.Cu") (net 2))
 (segment (start 94.35 79.8) (end 95.05 80.5) (width 0.2) (layer "F.Cu") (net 3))
 (segment (start 117.5 90) (end 106.1 90) (width 1.4) (layer "F.Cu") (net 3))
 (segment (start 106.1 90) (end 105 91.1) (width 1.4) (layer "F.Cu") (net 3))
 (segment (start 98.65 97.45) (end 105 91.1) (width 1.4) (layer "F.Cu") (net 3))
 (segment (start 92.5 97.45) (end 98.65 97.45) (width 1.4) (layer "F.Cu") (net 3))
 (segment (start 105 91.1) (end 95.05 81.15) (width 1.4) (layer "F.Cu") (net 3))
 (segment (start 94.35 76.8) (end 94.35 79.8) (width 0.2) (layer "F.Cu") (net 3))
 (segment (start 95.05 81.15) (end 95.05 80.5) (width 1.4) (layer "F.Cu") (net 3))
 (segment (start 96.1 89.9) (end 96.1 85.2) (width 1.4) (layer "F.Cu") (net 5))
 (segment (start 92.51 81.61) (end 92.51 80.5) (width 1.4) (layer "F.Cu") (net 5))
 (segment (start 96.1 85.2) (end 92.51 81.61) (width 1.4) (layer "F.Cu") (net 5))
 (segment (start 92.8 80.21) (end 92.51 80.5) (width 0.2) (layer "F.Cu") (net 5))
 (segment (start 91 95) (end 96.1 89.9) (width 1.4) (layer "F.Cu") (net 5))
 (segment (start 96.1 85.2) (end 88.7375 85.2) (width 1.4) (layer "F.Cu") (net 5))
 (segment (start 81.9 95) (end 91 95) (width 1.4) (layer "F.Cu") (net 5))
 (segment (start 80.7 91.5) (end 80.7 93.8) (width 1.4) (layer "F.Cu") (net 5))
 (segment (start 92.8 76.8) (end 92.8 80.21) (width 0.2) (layer "F.Cu") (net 5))
 (segment (start 88.7375 85.2) (end 86 82.4625) (width 1.4) (layer "F.Cu") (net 5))
 (segment (start 80.7 93.8) (end 81.9 95) (width 1.4) (layer "F.Cu") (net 5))
 (segment (start 77.3 89.216726) (end 77.3 95.2) (width 1.4) (layer "F.Cu") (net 1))
 (segment (start 91.75 88.3) (end 78.216726 88.3) (width 1.4) (layer "F.Cu") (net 1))
 (segment (start 77.3 91.5) (end 77.3 95.2) (width 1.4) (layer "F.Cu") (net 1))
 (segment (start 92.5 87.55) (end 91.75 88.3) (width 1.4) (layer "F.Cu") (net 1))
 (segment (start 78.216726 88.3) (end 77.3 89.216726) (width 1.4) (layer "F.Cu") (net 1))
 (segment (start 77.3 95.2) (end 75.5 97) (width 1.4) (layer "F.Cu") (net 1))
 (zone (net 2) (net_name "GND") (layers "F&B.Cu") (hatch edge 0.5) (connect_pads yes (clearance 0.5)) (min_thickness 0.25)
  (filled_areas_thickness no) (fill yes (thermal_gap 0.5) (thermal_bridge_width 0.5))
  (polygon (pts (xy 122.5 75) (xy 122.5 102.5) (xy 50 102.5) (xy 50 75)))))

